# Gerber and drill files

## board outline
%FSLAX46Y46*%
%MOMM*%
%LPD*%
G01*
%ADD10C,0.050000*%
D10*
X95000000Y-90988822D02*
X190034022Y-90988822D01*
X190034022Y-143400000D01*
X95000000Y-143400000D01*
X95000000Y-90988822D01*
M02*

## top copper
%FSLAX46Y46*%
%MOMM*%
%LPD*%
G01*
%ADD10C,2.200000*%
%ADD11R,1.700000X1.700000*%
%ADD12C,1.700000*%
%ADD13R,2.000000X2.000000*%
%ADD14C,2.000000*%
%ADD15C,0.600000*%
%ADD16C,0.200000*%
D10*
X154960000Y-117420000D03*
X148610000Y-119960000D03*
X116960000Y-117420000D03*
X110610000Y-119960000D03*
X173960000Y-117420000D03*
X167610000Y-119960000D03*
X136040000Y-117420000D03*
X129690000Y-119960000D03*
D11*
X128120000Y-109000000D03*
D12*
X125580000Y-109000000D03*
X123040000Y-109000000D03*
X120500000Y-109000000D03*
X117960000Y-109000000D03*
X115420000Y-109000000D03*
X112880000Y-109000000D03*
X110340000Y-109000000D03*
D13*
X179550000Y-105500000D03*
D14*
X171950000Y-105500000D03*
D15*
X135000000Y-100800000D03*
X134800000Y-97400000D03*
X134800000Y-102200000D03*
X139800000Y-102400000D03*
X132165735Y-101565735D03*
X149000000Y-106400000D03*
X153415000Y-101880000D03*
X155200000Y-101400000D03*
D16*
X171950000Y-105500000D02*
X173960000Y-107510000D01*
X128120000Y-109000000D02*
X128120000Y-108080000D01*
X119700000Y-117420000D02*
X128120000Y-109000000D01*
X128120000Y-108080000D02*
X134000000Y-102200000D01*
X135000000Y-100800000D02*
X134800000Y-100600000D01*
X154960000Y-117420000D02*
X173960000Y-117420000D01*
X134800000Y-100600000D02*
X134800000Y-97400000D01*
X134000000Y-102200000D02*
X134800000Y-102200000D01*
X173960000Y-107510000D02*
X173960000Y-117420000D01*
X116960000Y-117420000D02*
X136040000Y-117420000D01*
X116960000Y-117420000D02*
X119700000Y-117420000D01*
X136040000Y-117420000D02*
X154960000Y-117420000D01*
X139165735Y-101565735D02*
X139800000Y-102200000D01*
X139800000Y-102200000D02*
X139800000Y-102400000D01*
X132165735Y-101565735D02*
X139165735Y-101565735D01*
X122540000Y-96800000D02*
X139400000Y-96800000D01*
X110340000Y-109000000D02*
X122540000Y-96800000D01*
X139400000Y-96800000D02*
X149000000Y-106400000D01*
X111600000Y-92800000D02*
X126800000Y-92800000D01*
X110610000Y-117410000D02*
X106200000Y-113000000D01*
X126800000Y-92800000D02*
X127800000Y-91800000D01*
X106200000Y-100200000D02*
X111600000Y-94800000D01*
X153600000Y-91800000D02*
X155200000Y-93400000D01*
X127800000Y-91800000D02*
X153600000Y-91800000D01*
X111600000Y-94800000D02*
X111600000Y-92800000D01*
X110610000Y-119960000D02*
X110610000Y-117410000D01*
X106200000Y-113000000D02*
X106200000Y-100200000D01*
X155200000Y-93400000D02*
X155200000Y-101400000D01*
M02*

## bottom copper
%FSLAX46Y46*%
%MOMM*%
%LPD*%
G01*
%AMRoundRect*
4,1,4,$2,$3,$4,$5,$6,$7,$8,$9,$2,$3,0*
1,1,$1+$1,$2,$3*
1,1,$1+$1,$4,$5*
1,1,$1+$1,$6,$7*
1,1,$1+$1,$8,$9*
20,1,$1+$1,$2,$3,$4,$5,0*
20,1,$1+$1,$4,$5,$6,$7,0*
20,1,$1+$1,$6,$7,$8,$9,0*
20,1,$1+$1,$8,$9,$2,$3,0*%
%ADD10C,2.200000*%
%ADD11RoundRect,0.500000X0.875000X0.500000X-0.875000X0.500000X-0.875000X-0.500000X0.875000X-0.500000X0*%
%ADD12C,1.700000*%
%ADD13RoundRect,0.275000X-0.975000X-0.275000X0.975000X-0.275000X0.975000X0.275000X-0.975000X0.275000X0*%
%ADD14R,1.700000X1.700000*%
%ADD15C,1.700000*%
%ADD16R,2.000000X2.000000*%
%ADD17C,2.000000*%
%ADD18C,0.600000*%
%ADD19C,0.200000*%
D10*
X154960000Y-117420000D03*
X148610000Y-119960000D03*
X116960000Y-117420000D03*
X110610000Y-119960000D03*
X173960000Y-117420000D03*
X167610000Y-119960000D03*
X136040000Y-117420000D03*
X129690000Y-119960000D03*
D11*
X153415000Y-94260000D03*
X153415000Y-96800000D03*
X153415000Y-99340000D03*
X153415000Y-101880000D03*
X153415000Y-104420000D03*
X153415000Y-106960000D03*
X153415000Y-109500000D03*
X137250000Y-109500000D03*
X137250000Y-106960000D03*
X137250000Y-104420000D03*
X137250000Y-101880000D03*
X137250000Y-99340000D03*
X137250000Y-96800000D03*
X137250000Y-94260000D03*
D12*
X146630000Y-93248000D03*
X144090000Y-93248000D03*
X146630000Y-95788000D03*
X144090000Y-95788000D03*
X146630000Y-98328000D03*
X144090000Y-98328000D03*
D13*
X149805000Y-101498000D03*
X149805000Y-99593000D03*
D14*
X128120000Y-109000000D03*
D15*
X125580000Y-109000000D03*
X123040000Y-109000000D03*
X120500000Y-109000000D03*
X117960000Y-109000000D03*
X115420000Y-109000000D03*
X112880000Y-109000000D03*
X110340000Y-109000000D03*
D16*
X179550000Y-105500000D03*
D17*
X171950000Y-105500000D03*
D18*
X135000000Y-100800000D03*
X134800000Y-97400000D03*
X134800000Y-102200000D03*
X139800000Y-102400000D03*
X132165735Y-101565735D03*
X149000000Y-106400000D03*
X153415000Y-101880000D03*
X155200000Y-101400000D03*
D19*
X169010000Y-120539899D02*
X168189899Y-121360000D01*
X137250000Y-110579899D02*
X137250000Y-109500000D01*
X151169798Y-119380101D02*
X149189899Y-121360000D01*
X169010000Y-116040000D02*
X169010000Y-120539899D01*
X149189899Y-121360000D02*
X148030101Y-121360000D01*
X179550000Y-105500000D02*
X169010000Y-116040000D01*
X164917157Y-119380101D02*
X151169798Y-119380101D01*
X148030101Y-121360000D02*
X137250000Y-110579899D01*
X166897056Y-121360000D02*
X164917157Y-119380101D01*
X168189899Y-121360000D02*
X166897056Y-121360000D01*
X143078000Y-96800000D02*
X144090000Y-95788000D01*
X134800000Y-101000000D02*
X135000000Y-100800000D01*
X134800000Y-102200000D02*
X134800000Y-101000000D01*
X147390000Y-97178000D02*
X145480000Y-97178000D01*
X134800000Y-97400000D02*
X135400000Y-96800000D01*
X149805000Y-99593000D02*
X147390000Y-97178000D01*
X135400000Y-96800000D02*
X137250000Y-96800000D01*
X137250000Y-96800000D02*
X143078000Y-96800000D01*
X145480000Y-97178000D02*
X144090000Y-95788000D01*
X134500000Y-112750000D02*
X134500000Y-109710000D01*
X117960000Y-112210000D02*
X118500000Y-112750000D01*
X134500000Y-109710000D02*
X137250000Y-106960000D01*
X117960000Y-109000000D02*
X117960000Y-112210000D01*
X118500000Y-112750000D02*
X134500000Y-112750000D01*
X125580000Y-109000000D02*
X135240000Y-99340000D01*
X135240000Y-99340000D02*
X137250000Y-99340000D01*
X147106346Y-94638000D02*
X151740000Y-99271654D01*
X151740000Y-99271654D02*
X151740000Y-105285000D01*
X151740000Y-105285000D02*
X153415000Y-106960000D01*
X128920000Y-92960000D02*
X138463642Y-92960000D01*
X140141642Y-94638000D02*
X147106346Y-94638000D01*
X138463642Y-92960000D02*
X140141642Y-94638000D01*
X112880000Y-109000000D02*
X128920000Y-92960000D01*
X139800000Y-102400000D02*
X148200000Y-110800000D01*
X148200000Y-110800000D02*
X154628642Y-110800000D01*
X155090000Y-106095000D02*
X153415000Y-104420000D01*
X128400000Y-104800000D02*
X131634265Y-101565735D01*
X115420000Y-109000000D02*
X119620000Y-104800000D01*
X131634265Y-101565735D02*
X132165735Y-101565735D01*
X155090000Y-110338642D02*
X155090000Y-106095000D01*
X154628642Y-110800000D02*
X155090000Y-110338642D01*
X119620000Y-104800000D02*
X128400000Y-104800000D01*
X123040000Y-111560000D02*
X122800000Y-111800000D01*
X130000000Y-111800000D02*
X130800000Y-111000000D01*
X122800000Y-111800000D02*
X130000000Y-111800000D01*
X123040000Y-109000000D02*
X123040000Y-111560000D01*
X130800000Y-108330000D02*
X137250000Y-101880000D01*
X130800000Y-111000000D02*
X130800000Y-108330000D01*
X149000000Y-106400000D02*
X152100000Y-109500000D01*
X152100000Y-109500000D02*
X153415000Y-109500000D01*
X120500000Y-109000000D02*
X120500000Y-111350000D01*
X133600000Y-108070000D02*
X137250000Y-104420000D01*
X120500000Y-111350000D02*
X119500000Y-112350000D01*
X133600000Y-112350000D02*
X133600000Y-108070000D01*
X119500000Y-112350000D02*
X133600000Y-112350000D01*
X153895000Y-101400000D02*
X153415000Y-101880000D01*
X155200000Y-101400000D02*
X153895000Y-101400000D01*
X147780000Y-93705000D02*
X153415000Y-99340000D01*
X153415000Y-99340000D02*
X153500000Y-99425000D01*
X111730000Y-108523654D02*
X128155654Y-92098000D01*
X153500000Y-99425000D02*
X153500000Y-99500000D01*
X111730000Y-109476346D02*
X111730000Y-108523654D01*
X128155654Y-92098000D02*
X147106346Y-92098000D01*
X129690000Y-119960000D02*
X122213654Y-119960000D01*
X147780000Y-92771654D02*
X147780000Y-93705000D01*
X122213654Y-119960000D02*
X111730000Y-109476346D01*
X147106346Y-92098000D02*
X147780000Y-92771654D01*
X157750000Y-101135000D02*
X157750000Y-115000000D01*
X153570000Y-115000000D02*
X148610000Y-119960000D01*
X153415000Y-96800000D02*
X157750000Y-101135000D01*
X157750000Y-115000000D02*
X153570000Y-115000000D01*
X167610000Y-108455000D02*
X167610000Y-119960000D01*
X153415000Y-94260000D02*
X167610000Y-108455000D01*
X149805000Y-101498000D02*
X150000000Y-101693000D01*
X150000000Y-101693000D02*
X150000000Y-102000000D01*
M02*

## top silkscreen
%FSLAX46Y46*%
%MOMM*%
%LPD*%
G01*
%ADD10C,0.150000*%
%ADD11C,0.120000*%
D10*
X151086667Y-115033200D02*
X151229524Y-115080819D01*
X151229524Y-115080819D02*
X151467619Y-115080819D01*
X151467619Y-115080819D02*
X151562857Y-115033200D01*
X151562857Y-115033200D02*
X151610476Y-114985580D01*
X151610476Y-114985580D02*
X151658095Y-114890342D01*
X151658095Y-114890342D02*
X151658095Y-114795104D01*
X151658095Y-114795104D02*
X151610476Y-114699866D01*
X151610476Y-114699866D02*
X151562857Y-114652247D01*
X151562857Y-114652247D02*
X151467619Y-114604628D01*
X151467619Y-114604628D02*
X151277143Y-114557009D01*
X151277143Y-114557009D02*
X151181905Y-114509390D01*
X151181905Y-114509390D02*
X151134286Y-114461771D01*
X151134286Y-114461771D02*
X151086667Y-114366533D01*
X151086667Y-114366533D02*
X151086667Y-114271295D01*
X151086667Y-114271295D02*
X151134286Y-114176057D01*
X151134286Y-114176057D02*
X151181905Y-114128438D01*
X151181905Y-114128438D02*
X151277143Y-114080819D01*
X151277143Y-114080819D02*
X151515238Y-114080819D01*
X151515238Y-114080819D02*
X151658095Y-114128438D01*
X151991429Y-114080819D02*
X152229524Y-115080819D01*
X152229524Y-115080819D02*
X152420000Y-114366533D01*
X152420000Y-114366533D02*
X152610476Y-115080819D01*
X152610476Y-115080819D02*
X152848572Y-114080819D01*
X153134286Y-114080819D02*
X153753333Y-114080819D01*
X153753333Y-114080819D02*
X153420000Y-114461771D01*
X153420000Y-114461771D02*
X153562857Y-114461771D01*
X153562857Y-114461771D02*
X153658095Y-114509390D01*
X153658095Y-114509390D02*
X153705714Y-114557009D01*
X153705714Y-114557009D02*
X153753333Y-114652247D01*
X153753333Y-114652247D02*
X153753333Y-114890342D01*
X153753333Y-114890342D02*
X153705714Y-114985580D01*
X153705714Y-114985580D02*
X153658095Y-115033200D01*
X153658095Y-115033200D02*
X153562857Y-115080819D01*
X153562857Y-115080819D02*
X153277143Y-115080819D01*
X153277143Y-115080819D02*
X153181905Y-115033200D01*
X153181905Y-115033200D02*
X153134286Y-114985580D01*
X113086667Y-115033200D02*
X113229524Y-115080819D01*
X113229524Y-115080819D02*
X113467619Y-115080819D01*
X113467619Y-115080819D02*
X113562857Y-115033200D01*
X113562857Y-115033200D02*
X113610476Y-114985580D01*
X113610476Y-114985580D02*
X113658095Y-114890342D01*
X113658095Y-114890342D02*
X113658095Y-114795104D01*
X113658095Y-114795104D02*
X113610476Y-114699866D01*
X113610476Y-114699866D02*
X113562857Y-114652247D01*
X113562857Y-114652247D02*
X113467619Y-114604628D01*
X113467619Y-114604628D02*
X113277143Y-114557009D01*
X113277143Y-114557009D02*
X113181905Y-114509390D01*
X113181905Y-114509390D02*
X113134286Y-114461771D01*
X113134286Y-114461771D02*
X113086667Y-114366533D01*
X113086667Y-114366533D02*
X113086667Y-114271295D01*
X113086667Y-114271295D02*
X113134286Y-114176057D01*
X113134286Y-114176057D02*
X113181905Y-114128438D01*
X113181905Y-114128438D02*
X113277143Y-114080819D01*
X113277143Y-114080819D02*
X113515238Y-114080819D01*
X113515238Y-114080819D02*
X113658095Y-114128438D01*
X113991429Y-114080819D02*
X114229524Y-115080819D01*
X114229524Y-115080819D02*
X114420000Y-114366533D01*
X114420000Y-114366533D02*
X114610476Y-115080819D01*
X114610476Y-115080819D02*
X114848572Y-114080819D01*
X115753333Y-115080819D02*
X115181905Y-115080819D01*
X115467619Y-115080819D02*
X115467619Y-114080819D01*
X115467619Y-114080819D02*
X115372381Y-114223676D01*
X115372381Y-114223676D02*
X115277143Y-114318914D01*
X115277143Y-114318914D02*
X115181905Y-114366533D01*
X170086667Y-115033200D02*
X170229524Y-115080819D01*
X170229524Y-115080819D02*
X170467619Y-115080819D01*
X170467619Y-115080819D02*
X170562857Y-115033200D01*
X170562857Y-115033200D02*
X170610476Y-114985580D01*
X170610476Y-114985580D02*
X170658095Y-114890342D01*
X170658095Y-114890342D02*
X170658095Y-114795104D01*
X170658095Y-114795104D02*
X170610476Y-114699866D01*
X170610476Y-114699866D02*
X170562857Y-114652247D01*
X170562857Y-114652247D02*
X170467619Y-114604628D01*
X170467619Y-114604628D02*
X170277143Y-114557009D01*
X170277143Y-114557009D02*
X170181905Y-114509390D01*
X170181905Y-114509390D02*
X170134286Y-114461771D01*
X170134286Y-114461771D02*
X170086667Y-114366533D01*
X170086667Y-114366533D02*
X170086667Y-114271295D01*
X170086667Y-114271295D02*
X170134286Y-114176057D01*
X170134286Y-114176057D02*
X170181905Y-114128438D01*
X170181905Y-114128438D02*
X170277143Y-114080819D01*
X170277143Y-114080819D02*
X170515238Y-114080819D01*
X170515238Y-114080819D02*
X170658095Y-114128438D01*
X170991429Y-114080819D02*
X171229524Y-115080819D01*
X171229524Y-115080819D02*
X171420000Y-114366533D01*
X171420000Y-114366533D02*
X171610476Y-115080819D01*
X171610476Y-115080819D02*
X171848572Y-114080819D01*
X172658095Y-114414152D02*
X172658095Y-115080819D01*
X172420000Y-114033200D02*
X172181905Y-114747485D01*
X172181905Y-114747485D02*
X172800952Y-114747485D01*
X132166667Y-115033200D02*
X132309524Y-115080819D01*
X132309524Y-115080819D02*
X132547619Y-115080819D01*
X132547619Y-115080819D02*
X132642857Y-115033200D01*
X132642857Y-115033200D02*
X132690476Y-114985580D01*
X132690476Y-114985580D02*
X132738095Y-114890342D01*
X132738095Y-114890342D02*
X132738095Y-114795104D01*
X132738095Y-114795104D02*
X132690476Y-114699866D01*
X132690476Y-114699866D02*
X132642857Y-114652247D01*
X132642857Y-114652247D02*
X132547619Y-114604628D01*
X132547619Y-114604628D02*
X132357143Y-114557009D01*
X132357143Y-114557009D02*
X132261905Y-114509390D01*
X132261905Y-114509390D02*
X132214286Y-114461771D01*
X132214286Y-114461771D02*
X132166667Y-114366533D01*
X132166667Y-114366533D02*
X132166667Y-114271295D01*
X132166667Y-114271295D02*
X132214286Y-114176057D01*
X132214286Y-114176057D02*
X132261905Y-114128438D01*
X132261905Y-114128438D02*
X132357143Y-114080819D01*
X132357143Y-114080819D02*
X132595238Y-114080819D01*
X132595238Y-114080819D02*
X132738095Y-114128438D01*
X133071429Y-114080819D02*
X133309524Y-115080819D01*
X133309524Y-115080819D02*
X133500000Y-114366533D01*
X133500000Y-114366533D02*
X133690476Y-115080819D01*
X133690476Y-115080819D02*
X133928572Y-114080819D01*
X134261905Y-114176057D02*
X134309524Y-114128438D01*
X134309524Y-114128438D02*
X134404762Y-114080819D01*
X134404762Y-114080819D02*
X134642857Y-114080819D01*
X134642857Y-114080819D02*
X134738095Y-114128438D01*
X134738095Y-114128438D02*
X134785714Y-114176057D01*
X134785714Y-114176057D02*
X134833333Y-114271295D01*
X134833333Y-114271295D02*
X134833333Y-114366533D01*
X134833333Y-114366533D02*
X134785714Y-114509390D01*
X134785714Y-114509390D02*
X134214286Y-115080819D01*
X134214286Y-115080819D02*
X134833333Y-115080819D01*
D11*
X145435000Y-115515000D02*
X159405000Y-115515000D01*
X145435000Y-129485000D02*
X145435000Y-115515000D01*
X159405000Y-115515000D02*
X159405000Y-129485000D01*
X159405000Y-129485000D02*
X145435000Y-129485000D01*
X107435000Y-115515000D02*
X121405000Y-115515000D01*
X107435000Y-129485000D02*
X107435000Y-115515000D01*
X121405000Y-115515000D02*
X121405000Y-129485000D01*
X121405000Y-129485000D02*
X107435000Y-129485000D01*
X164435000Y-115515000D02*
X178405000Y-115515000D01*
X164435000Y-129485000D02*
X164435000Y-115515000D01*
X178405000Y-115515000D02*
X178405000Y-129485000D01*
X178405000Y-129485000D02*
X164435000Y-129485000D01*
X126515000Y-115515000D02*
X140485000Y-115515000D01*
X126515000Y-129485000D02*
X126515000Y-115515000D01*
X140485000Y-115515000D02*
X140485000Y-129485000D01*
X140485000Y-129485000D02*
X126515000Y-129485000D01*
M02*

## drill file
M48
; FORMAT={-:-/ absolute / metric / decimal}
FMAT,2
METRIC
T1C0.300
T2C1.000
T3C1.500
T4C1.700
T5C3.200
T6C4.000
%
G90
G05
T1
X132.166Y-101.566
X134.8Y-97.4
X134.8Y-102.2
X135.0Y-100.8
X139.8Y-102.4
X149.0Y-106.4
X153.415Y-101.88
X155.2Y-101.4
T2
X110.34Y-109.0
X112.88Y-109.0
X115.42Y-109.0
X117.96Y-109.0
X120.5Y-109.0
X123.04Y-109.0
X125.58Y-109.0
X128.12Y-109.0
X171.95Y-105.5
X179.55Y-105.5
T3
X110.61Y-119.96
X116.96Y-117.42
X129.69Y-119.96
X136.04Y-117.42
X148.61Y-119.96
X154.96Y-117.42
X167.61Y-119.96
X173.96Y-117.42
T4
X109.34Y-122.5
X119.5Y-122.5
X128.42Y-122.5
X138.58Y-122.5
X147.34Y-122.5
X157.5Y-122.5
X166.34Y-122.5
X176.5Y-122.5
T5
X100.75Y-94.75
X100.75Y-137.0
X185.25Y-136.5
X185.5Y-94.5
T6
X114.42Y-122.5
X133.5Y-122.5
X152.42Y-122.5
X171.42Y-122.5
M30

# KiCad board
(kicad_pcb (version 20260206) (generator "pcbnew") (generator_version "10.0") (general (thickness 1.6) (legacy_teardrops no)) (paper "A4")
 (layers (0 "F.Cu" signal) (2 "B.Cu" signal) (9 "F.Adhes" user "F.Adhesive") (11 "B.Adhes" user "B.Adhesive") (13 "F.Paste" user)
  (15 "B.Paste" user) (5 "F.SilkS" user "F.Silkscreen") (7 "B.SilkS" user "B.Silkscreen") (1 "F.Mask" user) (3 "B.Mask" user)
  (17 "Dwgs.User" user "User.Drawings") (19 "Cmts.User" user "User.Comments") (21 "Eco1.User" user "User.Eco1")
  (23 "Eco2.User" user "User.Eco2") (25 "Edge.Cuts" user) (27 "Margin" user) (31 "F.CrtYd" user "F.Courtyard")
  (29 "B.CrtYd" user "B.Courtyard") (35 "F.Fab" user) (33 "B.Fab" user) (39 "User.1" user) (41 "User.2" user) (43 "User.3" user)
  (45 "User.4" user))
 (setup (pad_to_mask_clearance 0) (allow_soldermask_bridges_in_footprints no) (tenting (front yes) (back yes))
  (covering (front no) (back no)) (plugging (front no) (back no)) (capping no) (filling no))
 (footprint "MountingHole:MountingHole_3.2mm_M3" (layer "F.Cu") (at 185.25 136.5)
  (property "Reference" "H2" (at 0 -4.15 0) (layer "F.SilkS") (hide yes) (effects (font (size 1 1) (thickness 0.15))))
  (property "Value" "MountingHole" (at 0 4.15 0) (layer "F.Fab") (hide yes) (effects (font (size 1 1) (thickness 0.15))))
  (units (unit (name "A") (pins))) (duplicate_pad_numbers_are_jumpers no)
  (pad "" np_thru_hole circle (at 0 0) (size 3.2 3.2) (drill 3.2) (layers "*.Cu" "*.Mask")))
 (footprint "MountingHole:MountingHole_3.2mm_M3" (layer "F.Cu") (at 100.75 137)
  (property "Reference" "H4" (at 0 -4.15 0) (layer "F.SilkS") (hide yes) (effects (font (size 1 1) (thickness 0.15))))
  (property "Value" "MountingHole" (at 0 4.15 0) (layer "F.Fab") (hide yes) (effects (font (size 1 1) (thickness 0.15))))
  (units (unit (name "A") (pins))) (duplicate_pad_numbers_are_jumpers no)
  (pad "" np_thru_hole circle (at 0 0) (size 3.2 3.2) (drill 3.2) (layers "*.Cu" "*.Mask")))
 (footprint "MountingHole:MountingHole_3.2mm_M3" (layer "F.Cu") (at 185.5 94.5)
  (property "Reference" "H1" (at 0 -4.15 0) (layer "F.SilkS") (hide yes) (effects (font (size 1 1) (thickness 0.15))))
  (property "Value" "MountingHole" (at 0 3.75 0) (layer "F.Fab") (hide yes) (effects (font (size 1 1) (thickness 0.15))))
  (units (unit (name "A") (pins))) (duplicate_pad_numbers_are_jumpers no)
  (pad "" np_thru_hole circle (at 0 0) (size 3.2 3.2) (drill 3.2) (layers "*.Cu" "*.Mask")))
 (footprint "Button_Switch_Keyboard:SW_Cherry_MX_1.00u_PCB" (layer "F.Cu") (at 154.96 117.42)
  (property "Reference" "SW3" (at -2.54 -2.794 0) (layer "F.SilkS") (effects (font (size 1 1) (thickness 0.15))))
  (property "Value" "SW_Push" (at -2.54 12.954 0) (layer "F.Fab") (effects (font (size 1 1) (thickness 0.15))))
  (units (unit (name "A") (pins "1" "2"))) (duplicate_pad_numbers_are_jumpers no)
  (fp_line (start -9.525 -1.905) (end 4.445 -1.905) (stroke (width 0.12) (type solid)) (layer "F.SilkS"))
  (fp_line (start -9.525 12.065) (end -9.525 -1.905) (stroke (width 0.12) (type solid)) (layer "F.SilkS"))
  (fp_line (start 4.445 -1.905) (end 4.445 12.065) (stroke (width 0.12) (type solid)) (layer "F.SilkS"))
  (fp_line (start 4.445 12.065) (end -9.525 12.065) (stroke (width 0.12) (type solid)) (layer "F.SilkS"))
  (pad "" np_thru_hole circle (at -7.62 5.08) (size 1.7 1.7) (drill 1.7) (layers "*.Cu" "*.Mask"))
  (pad "" np_thru_hole circle (at -2.54 5.08) (size 4 4) (drill 4) (layers "*.Cu" "*.Mask"))
  (pad "" np_thru_hole circle (at 2.54 5.08) (size 1.7 1.7) (drill 1.7) (layers "*.Cu" "*.Mask"))
  (pad "1" thru_hole circle (at 0 0) (size 2.2 2.2) (drill 1.5) (layers "*.Cu" "*.Mask") (remove_unused_layers no) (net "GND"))
  (pad "2" thru_hole circle (at -6.35 2.54) (size 2.2 2.2) (drill 1.5) (layers "*.Cu" "*.Mask") (remove_unused_layers no)
   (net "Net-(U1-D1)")))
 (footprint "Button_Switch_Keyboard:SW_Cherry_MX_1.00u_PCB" (layer "F.Cu") (at 116.96 117.42)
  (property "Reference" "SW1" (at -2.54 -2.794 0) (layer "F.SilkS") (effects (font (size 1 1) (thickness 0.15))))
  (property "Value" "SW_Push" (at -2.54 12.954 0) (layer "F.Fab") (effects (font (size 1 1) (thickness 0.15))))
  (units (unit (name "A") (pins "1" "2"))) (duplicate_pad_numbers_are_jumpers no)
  (fp_line (start -9.525 -1.905) (end 4.445 -1.905) (stroke (width 0.12) (type solid)) (layer "F.SilkS"))
  (fp_line (start -9.525 12.065) (end -9.525 -1.905) (stroke (width 0.12) (type solid)) (layer "F.SilkS"))
  (fp_line (start 4.445 -1.905) (end 4.445 12.065) (stroke (width 0.12) (type solid)) (layer "F.SilkS"))
  (fp_line (start 4.445 12.065) (end -9.525 12.065) (stroke (width 0.12) (type solid)) (layer "F.SilkS"))
  (pad "" np_thru_hole circle (at -7.62 5.08) (size 1.7 1.7) (drill 1.7) (layers "*.Cu" "*.Mask"))
  (pad "" np_thru_hole circle (at -2.54 5.08) (size 4 4) (drill 4) (layers "*.Cu" "*.Mask"))
  (pad "" np_thru_hole circle (at 2.54 5.08) (size 1.7 1.7) (drill 1.7) (layers "*.Cu" "*.Mask"))
  (pad "1" thru_hole circle (at 0 0) (size 2.2 2.2) (drill 1.5) (layers "*.Cu" "*.Mask") (remove_unused_layers no) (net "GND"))
  (pad "2" thru_hole circle (at -6.35 2.54) (size 2.2 2.2) (drill 1.5) (layers "*.Cu" "*.Mask") (remove_unused_layers no)
   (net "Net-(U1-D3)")))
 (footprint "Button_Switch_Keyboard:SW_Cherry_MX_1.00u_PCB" (layer "F.Cu") (at 173.96 117.42)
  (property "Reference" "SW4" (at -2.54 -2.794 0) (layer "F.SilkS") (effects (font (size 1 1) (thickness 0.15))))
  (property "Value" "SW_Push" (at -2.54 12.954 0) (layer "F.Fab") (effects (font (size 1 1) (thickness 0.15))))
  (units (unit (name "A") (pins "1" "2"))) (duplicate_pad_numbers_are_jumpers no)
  (fp_line (start -9.525 -1.905) (end 4.445 -1.905) (stroke (width 0.12) (type solid)) (layer "F.SilkS"))
  (fp_line (start -9.525 12.065) (end -9.525 -1.905) (stroke (width 0.12) (type solid)) (layer "F.SilkS"))
  (fp_line (start 4.445 -1.905) (end 4.445 12.065) (stroke (width 0.12) (type solid)) (layer "F.SilkS"))
  (fp_line (start 4.445 12.065) (end -9.525 12.065) (stroke (width 0.12) (type solid)) (layer "F.SilkS"))
  (pad "" np_thru_hole circle (at -7.62 5.08) (size 1.7 1.7) (drill 1.7) (layers "*.Cu" "*.Mask"))
  (pad "" np_thru_hole circle (at -2.54 5.08) (size 4 4) (drill 4) (layers "*.Cu" "*.Mask"))
  (pad "" np_thru_hole circle (at 2.54 5.08) (size 1.7 1.7) (drill 1.7) (layers "*.Cu" "*.Mask"))
  (pad "1" thru_hole circle (at 0 0) (size 2.2 2.2) (drill 1.5) (layers "*.Cu" "*.Mask") (remove_unused_layers no) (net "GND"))
  (pad "2" thru_hole circle (at -6.35 2.54) (size 2.2 2.2) (drill 1.5) (layers "*.Cu" "*.Mask") (remove_unused_layers no)
   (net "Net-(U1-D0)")))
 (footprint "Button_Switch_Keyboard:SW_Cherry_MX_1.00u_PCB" (layer "F.Cu") (at 136.04 117.42)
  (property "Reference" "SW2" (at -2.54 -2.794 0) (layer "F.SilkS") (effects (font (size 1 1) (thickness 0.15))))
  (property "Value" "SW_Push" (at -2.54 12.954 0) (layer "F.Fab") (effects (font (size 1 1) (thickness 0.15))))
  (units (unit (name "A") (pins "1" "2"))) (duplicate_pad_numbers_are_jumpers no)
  (fp_line (start -9.525 -1.905) (end 4.445 -1.905) (stroke (width 0.12) (type solid)) (layer "F.SilkS"))
  (fp_line (start -9.525 12.065) (end -9.525 -1.905) (stroke (width 0.12) (type solid)) (layer "F.SilkS"))
  (fp_line (start 4.445 -1.905) (end 4.445 12.065) (stroke (width 0.12) (type solid)) (layer "F.SilkS"))
  (fp_line (start 4.445 12.065) (end -9.525 12.065) (stroke (width 0.12) (type solid)) (layer "F.SilkS"))
  (pad "" np_thru_hole circle (at -7.62 5.08) (size 1.7 1.7) (drill 1.7) (layers "*.Cu" "*.Mask"))
  (pad "" np_thru_hole circle (at -2.54 5.08) (size 4 4) (drill 4) (layers "*.Cu" "*.Mask"))
  (pad "" np_thru_hole circle (at 2.54 5.08) (size 1.7 1.7) (drill 1.7) (layers "*.Cu" "*.Mask"))
  (pad "1" thru_hole circle (at 0 0) (size 2.2 2.2) (drill 1.5) (layers "*.Cu" "*.Mask") (remove_unused_layers no) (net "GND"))
  (pad "2" thru_hole circle (at -6.35 2.54) (size 2.2 2.2) (drill 1.5) (layers "*.Cu" "*.Mask") (remove_unused_layers no)
   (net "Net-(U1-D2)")))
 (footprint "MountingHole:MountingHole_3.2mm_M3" (layer "F.Cu") (at 100.75 94.75)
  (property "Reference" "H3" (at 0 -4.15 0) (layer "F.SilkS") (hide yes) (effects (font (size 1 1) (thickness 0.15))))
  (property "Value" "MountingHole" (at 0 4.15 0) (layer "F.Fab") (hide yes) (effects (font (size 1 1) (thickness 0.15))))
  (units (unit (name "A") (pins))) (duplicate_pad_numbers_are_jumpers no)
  (pad "" np_thru_hole circle (at 0 0) (size 3.2 3.2) (drill 3.2) (layers "*.Cu" "*.Mask")))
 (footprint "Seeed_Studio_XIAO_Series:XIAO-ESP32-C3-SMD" (layer "B.Cu") (at 154.25 112.38 180)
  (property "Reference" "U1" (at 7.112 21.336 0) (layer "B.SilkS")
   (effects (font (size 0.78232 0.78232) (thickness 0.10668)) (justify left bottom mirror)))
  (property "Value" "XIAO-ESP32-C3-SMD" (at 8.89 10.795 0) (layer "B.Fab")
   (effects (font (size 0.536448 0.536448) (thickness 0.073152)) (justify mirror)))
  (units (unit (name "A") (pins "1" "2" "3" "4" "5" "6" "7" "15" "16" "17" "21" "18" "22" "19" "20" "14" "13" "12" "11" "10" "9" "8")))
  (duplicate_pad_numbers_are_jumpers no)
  (pad "1" smd roundrect (at 0.835 18.12 180) (size 2.75 2) (layers "B.Cu" "B.Mask" "B.Paste") (roundrect_rratio 0.25) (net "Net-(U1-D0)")
   (solder_mask_margin 0.0508) (thermal_bridge_angle 45))
  (pad "2" smd roundrect (at 0.835 15.58 180) (size 2.75 2) (layers "B.Cu" "B.Mask" "B.Paste") (roundrect_rratio 0.25) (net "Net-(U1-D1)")
   (solder_mask_margin 0.0508) (thermal_bridge_angle 45))
  (pad "3" smd roundrect (at 0.835 13.04 180) (size 2.75 2) (layers "B.Cu" "B.Mask" "B.Paste") (roundrect_rratio 0.25) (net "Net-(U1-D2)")
   (solder_mask_margin 0.0508) (thermal_bridge_angle 45))
  (pad "4" smd roundrect (at 0.835 10.5 180) (size 2.75 2) (layers "B.Cu" "B.Mask" "B.Paste") (roundrect_rratio 0.25) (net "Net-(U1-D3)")
   (solder_mask_margin 0.0508) (thermal_bridge_angle 45))
  (pad "5" smd roundrect (at 0.835 7.96 180) (size 2.75 2) (layers "B.Cu" "B.Mask" "B.Paste") (roundrect_rratio 0.25) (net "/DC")
   (solder_mask_margin 0.0508) (thermal_bridge_angle 45))
  (pad "6" smd roundrect (at 0.835 5.42 180) (size 2.75 2) (layers "B.Cu" "B.Mask" "B.Paste") (roundrect_rratio 0.25) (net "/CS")
   (solder_mask_margin 0.0508) (thermal_bridge_angle 45))
  (pad "7" smd roundrect (at 0.835 2.88 180) (size 2.75 2) (layers "B.Cu" "B.Mask" "B.Paste") (roundrect_rratio 0.25) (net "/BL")
   (solder_mask_margin 0.0508) (thermal_bridge_angle 45))
  (pad "8" smd roundrect (at 17 2.88 180) (size 2.75 2) (layers "B.Cu" "B.Mask" "B.Paste") (roundrect_rratio 0.25) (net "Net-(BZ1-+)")
   (solder_mask_margin 0.0508) (thermal_bridge_angle 45))
  (pad "9" smd roundrect (at 17 5.42 180) (size 2.75 2) (layers "B.Cu" "B.Mask" "B.Paste") (roundrect_rratio 0.25) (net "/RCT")
   (solder_mask_margin 0.0508) (thermal_bridge_angle 45))
  (pad "10" smd roundrect (at 17 7.96 180) (size 2.75 2) (layers "B.Cu" "B.Mask" "B.Paste") (roundrect_rratio 0.25) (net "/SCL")
   (solder_mask_margin 0.0508) (thermal_bridge_angle 45))
  (pad "11" smd roundrect (at 17 10.5 180) (size 2.75 2) (layers "B.Cu" "B.Mask" "B.Paste") (roundrect_rratio 0.25) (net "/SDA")
   (solder_mask_margin 0.0508) (thermal_bridge_angle 45))
  (pad "12" smd roundrect (at 17 13.04 180) (size 2.75 2) (layers "B.Cu" "B.Mask" "B.Paste") (roundrect_rratio 0.25) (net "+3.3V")
   (solder_mask_margin 0.0508) (thermal_bridge_angle 45))
  (pad "13" smd roundrect (at 17 15.58 180) (size 2.75 2) (layers "B.Cu" "B.Mask" "B.Paste") (roundrect_rratio 0.25) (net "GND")
   (solder_mask_margin 0.0508) (thermal_bridge_angle 45))
  (pad "14" smd roundrect (at 17 18.12 180) (size 2.75 2) (layers "B.Cu" "B.Mask" "B.Paste") (roundrect_rratio 0.25)
   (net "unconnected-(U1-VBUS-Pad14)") (solder_mask_margin 0.0508) (thermal_bridge_angle 45))
  (pad "15" smd circle (at 7.62 19.132 180) (size 1.7 1.7) (layers "B.Cu" "B.Mask" "B.Paste") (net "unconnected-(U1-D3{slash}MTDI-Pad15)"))
  (pad "16" smd circle (at 10.16 19.132 180) (size 1.7 1.7) (layers "B.Cu" "B.Mask" "B.Paste") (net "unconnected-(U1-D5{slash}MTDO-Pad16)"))
  (pad "17" smd circle (at 7.62 16.592 180) (size 1.7 1.7) (layers "B.Cu" "B.Mask" "B.Paste") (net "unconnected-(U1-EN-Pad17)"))
  (pad "18" smd circle (at 10.16 16.592 180) (size 1.7 1.7) (layers "B.Cu" "B.Mask" "B.Paste") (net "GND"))
  (pad "19" smd circle (at 7.62 14.052 180) (size 1.7 1.7) (layers "B.Cu" "B.Mask" "B.Paste") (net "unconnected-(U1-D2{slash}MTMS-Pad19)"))
  (pad "20" smd circle (at 10.16 14.052 180) (size 1.7 1.7) (layers "B.Cu" "B.Mask" "B.Paste") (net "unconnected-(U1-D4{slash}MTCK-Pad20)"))
  (pad "21" smd roundrect (at 4.445 10.882) (size 2.5 1.1) (layers "B.Cu" "B.Mask" "B.Paste") (roundrect_rratio 0.25)
   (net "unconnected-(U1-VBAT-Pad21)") (thermal_bridge_angle 45))
  (pad "22" smd roundrect (at 4.445 12.787) (size 2.5 1.1) (layers "B.Cu" "B.Mask" "B.Paste") (roundrect_rratio 0.25) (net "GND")
   (thermal_bridge_angle 45)))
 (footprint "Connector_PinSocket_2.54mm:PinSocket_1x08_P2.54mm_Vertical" (layer "B.Cu") (at 128.12 109 90)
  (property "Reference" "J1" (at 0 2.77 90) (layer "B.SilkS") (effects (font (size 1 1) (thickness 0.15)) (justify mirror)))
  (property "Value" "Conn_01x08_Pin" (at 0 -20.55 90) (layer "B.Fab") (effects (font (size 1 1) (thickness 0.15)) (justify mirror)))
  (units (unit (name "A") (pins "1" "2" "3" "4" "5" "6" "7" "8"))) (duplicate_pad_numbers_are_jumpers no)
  (pad "1" thru_hole rect (at 0 0 90) (size 1.7 1.7) (drill 1) (layers "*.Cu" "*.Mask") (remove_unused_layers no) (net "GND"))
  (pad "2" thru_hole circle (at 0 -2.54 90) (size 1.7 1.7) (drill 1) (layers "*.Cu" "*.Mask") (remove_unused_layers no) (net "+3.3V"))
  (pad "3" thru_hole circle (at 0 -5.08 90) (size 1.7 1.7) (drill 1) (layers "*.Cu" "*.Mask") (remove_unused_layers no) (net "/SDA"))
  (pad "4" thru_hole circle (at 0 -7.62 90) (size 1.7 1.7) (drill 1) (layers "*.Cu" "*.Mask") (remove_unused_layers no) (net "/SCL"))
  (pad "5" thru_hole circle (at 0 -10.16 90) (size 1.7 1.7) (drill 1) (layers "*.Cu" "*.Mask") (remove_unused_layers no) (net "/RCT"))
  (pad "6" thru_hole circle (at 0 -12.7 90) (size 1.7 1.7) (drill 1) (layers "*.Cu" "*.Mask") (remove_unused_layers no) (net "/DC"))
  (pad "7" thru_hole circle (at 0 -15.24 90) (size 1.7 1.7) (drill 1) (layers "*.Cu" "*.Mask") (remove_unused_layers no) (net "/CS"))
  (pad "8" thru_hole circle (at 0 -17.78 90) (size 1.7 1.7) (drill 1) (layers "*.Cu" "*.Mask") (remove_unused_layers no) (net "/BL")))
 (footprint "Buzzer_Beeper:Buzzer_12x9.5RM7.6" (layer "B.Cu") (at 179.55 105.5 180)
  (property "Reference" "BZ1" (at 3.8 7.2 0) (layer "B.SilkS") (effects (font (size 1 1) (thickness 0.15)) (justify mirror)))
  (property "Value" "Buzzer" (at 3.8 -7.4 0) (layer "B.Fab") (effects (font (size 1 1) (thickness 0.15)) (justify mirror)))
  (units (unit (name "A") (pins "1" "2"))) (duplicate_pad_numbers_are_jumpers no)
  (pad "1" thru_hole rect (at 0 0 180) (size 2 2) (drill 1) (layers "*.Cu" "*.Mask") (remove_unused_layers no) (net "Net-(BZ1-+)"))
  (pad "2" thru_hole circle (at 7.6 0 180) (size 2 2) (drill 1) (layers "*.Cu" "*.Mask") (remove_unused_layers no) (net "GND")))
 (gr_rect (start 95 90.988822) (end 190.034022 143.4) (stroke (width 0.05) (type default)) (fill no) (layer "Edge.Cuts"))
 (segment (start 169.01 120.539899) (end 168.189899 121.36) (width 0.2) (layer "B.Cu") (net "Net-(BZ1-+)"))
 (segment (start 137.25 110.579899) (end 137.25 109.5) (width 0.2) (layer "B.Cu") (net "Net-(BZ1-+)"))
 (segment (start 151.169798 119.380101) (end 149.189899 121.36) (width 0.2) (layer "B.Cu") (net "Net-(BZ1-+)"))
 (segment (start 169.01 116.04) (end 169.01 120.539899) (width 0.2) (layer "B.Cu") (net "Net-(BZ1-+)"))
 (segment (start 149.189899 121.36) (end 148.030101 121.36) (width 0.2) (layer "B.Cu") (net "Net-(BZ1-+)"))
 (segment (start 179.55 105.5) (end 169.01 116.04) (width 0.2) (layer "B.Cu") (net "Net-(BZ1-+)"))
 (segment (start 164.917157 119.380101) (end 151.169798 119.380101) (width 0.2) (layer "B.Cu") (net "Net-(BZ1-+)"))
 (segment (start 148.030101 121.36) (end 137.25 110.579899) (width 0.2) (layer "B.Cu") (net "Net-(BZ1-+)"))
 (segment (start 166.897056 121.36) (end 164.917157 119.380101) (width 0.2) (layer "B.Cu") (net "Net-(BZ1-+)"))
 (segment (start 168.189899 121.36) (end 166.897056 121.36) (width 0.2) (layer "B.Cu") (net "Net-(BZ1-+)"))
 (segment (start 171.95 105.5) (end 173.96 107.51) (width 0.2) (layer "F.Cu") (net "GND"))
 (segment (start 128.12 109) (end 128.12 108.08) (width 0.2) (layer "F.Cu") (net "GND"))
 (segment (start 119.7 117.42) (end 128.12 109) (width 0.2) (layer "F.Cu") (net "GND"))
 (segment (start 128.12 108.08) (end 134 102.2) (width 0.2) (layer "F.Cu") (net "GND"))
 (segment (start 135 100.8) (end 134.8 100.6) (width 0.2) (layer "F.Cu") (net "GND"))
 (segment (start 154.96 117.42) (end 173.96 117.42) (width 0.2) (layer "F.Cu") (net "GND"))
 (segment (start 134.8 100.6) (end 134.8 97.4) (width 0.2) (layer "F.Cu") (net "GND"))
 (segment (start 134 102.2) (end 134.8 102.2) (width 0.2) (layer "F.Cu") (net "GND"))
 (segment (start 173.96 107.51) (end 173.96 117.42) (width 0.2) (layer "F.Cu") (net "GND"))
 (segment (start 116.96 117.42) (end 136.04 117.42) (width 0.2) (layer "F.Cu") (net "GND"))
 (segment (start 116.96 117.42) (end 119.7 117.42) (width 0.2) (layer "F.Cu") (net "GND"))
 (segment (start 136.04 117.42) (end 154.96 117.42) (width 0.2) (layer "F.Cu") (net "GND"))
 (via (at 135 100.8) (size 0.6) (drill 0.3) (layers "F.Cu" "B.Cu") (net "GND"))
 (via (at 134.8 97.4) (size 0.6) (drill 0.3) (layers "F.Cu" "B.Cu") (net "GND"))
 (via (at 134.8 102.2) (size 0.6) (drill 0.3) (layers "F.Cu" "B.Cu") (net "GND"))
 (segment (start 143.078 96.8) (end 144.09 95.788) (width 0.2) (layer "B.Cu") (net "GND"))
 (segment (start 134.8 101) (end 135 100.8) (width 0.2) (layer "B.Cu") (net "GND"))
 (segment (start 134.8 102.2) (end 134.8 101) (width 0.2) (layer "B.Cu") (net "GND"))
 (segment (start 147.39 97.178) (end 145.48 97.178) (width 0.2) (layer "B.Cu") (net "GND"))
 (segment (start 134.8 97.4) (end 135.4 96.8) (width 0.2) (layer "B.Cu") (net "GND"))
 (segment (start 149.805 99.593) (end 147.39 97.178) (width 0.2) (layer "B.Cu") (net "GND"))
 (segment (start 135.4 96.8) (end 137.25 96.8) (width 0.2) (layer "B.Cu") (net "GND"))
 (segment (start 137.25 96.8) (end 143.078 96.8) (width 0.2) (layer "B.Cu") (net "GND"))
 (segment (start 145.48 97.178) (end 144.09 95.788) (width 0.2) (layer "B.Cu") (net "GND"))
 (segment (start 134.5 112.75) (end 134.5 109.71) (width 0.2) (layer "B.Cu") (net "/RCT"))
 (segment (start 117.96 112.21) (end 118.5 112.75) (width 0.2) (layer "B.Cu") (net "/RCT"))
 (segment (start 134.5 109.71) (end 137.25 106.96) (width 0.2) (layer "B.Cu") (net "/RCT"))
 (segment (start 117.96 109) (end 117.96 112.21) (width 0.2) (layer "B.Cu") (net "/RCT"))
 (segment (start 118.5 112.75) (end 134.5 112.75) (width 0.2) (layer "B.Cu") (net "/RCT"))
 (segment (start 125.58 109) (end 135.24 99.34) (width 0.2) (layer "B.Cu") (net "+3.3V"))
 (segment (start 135.24 99.34) (end 137.25 99.34) (width 0.2) (layer "B.Cu") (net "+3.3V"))
 (segment (start 147.106346 94.638) (end 151.74 99.271654) (width 0.2) (layer "B.Cu") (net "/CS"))
 (segment (start 151.74 99.271654) (end 151.74 105.285) (width 0.2) (layer "B.Cu") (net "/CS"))
 (segment (start 151.74 105.285) (end 153.415 106.96) (width 0.2) (layer "B.Cu") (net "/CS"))
 (segment (start 128.92 92.96) (end 138.463642 92.96) (width 0.2) (layer "B.Cu") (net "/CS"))
 (segment (start 140.141642 94.638) (end 147.106346 94.638) (width 0.2) (layer "B.Cu") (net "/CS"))
 (segment (start 138.463642 92.96) (end 140.141642 94.638) (width 0.2) (layer "B.Cu") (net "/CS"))
 (segment (start 112.88 109) (end 128.92 92.96) (width 0.2) (layer "B.Cu") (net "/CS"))
 (segment (start 139.165735 101.565735) (end 139.8 102.2) (width 0.2) (layer "F.Cu") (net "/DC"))
 (segment (start 139.8 102.2) (end 139.8 102.4) (width 0.2) (layer "F.Cu") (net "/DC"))
 (segment (start 132.165735 101.565735) (end 139.165735 101.565735) (width 0.2) (layer "F.Cu") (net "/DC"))
 (via (at 139.8 102.4) (size 0.6) (drill 0.3) (layers "F.Cu" "B.Cu") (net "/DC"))
 (via (at 132.165735 101.565735) (size 0.6) (drill 0.3) (layers "F.Cu" "B.Cu") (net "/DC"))
 (segment (start 139.8 102.4) (end 148.2 110.8) (width 0.2) (layer "B.Cu") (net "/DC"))
 (segment (start 148.2 110.8) (end 154.628642 110.8) (width 0.2) (layer "B.Cu") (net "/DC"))
 (segment (start 155.09 106.095) (end 153.415 104.42) (width 0.2) (layer "B.Cu") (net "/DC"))
 (segment (start 128.4 104.8) (end 131.634265 101.565735) (width 0.2) (layer "B.Cu") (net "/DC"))
 (segment (start 115.42 109) (end 119.62 104.8) (width 0.2) (layer "B.Cu") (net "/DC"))
 (segment (start 131.634265 101.565735) (end 132.165735 101.565735) (width 0.2) (layer "B.Cu") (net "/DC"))
 (segment (start 155.09 110.338642) (end 155.09 106.095) (width 0.2) (layer "B.Cu") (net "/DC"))
 (segment (start 154.628642 110.8) (end 155.09 110.338642) (width 0.2) (layer "B.Cu") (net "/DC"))
 (segment (start 119.62 104.8) (end 128.4 104.8) (width 0.2) (layer "B.Cu") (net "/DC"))
 (segment (start 123.04 111.56) (end 122.8 111.8) (width 0.2) (layer "B.Cu") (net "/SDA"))
 (segment (start 130 111.8) (end 130.8 111) (width 0.2) (layer "B.Cu") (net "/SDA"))
 (segment (start 122.8 111.8) (end 130 111.8) (width 0.2) (layer "B.Cu") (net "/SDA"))
 (segment (start 123.04 109) (end 123.04 111.56) (width 0.2) (layer "B.Cu") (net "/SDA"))
 (segment (start 130.8 108.33) (end 137.25 101.88) (width 0.2) (layer "B.Cu") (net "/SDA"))
 (segment (start 130.8 111) (end 130.8 108.33) (width 0.2) (layer "B.Cu") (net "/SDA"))
 (segment (start 122.54 96.8) (end 139.4 96.8) (width 0.2) (layer "F.Cu") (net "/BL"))
 (segment (start 110.34 109) (end 122.54 96.8) (width 0.2) (layer "F.Cu") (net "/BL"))
 (segment (start 139.4 96.8) (end 149 106.4) (width 0.2) (layer "F.Cu") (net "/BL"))
 (via (at 149 106.4) (size 0.6) (drill 0.3) (layers "F.Cu" "B.Cu") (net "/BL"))
 (segment (start 149 106.4) (end 152.1 109.5) (width 0.2) (layer "B.Cu") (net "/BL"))
 (segment (start 152.1 109.5) (end 153.415 109.5) (width 0.2) (layer "B.Cu") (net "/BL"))
 (segment (start 120.5 109) (end 120.5 111.35) (width 0.2) (layer "B.Cu") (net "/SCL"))
 (segment (start 133.6 108.07) (end 137.25 104.42) (width 0.2) (layer "B.Cu") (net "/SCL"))
 (segment (start 120.5 111.35) (end 119.5 112.35) (width 0.2) (layer "B.Cu") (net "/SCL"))
 (segment (start 133.6 112.35) (end 133.6 108.07) (width 0.2) (layer "B.Cu") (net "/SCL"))
 (segment (start 119.5 112.35) (end 133.6 112.35) (width 0.2) (layer "B.Cu") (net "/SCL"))
 (segment (start 111.6 92.8) (end 126.8 92.8) (width 0.2) (layer "F.Cu") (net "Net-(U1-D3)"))
 (segment (start 110.61 117.41) (end 106.2 113) (width 0.2) (layer "F.Cu") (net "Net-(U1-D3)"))
 (segment (start 126.8 92.8) (end 127.8 91.8) (width 0.2) (layer "F.Cu") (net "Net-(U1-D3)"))
 (segment (start 106.2 100.2) (end 111.6 94.8) (width 0.2) (layer "F.Cu") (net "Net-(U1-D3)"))
 (segment (start 153.6 91.8) (end 155.2 93.4) (width 0.2) (layer "F.Cu") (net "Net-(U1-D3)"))
 (segment (start 127.8 91.8) (end 153.6 91.8) (width 0.2) (layer "F.Cu") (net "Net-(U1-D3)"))
 (segment (start 111.6 94.8) (end 111.6 92.8) (width 0.2) (layer "F.Cu") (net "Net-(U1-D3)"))
 (segment (start 110.61 119.96) (end 110.61 117.41) (width 0.2) (layer "F.Cu") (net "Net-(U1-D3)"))
 (segment (start 106.2 113) (end 106.2 100.2) (width 0.2) (layer "F.Cu") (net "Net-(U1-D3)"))
 (segment (start 155.2 93.4) (end 155.2 101.4) (width 0.2) (layer "F.Cu") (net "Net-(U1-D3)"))
 (via (at 153.415 101.88) (size 0.6) (drill 0.3) (layers "F.Cu" "B.Cu") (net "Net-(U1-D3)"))
 (via (at 155.2 101.4) (size 0.6) (drill 0.3) (layers "F.Cu" "B.Cu") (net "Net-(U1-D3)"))
 (segment (start 153.895 101.4) (end 153.415 101.88) (width 0.2) (layer "B.Cu") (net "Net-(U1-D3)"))
 (segment (start 155.2 101.4) (end 153.895 101.4) (width 0.2) (layer "B.Cu") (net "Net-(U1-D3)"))
 (segment (start 147.78 93.705) (end 153.415 99.34) (width 0.2) (layer "B.Cu") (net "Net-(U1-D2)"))
 (segment (start 153.415 99.34) (end 153.5 99.425) (width 0.2) (layer "B.Cu") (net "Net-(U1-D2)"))
 (segment (start 111.73 108.523654) (end 128.155654 92.098) (width 0.2) (layer "B.Cu") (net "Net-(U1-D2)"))
 (segment (start 153.5 99.425) (end 153.5 99.5) (width 0.2) (layer "B.Cu") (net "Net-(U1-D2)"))
 (segment (start 111.73 109.476346) (end 111.73 108.523654) (width 0.2) (layer "B.Cu") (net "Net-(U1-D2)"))
 (segment (start 128.155654 92.098) (end 147.106346 92.098) (width 0.2) (layer "B.Cu") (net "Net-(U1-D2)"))
 (segment (start 129.69 119.96) (end 122.213654 119.96) (width 0.2) (layer "B.Cu") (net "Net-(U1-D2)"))
 (segment (start 147.78 92.771654) (end 147.78 93.705) (width 0.2) (layer "B.Cu") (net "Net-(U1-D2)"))
 (segment (start 122.213654 119.96) (end 111.73 109.476346) (width 0.2) (layer "B.Cu") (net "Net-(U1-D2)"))
 (segment (start 147.106346 92.098) (end 147.78 92.771654) (width 0.2) (layer "B.Cu") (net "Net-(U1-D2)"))
 (segment (start 157.75 101.135) (end 157.75 115) (width 0.2) (layer "B.Cu") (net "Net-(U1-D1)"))
 (segment (start 153.57 115) (end 148.61 119.96) (width 0.2) (layer "B.Cu") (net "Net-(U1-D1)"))
 (segment (start 153.415 96.8) (end 157.75 101.135) (width 0.2) (layer "B.Cu") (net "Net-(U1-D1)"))
 (segment (start 157.75 115) (end 153.57 115) (width 0.2) (layer "B.Cu") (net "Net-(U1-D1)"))
 (segment (start 167.61 108.455) (end 167.61 119.96) (width 0.2) (layer "B.Cu") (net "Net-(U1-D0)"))
 (segment (start 153.415 94.26) (end 167.61 108.455) (width 0.2) (layer "B.Cu") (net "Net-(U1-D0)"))
 (segment (start 149.805 101.498) (end 150 101.693) (width 0.2) (layer "B.Cu") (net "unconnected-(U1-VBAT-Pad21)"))
 (segment (start 150 101.693) (end 150 102) (width 0.2) (layer "B.Cu") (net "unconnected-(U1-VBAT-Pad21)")))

